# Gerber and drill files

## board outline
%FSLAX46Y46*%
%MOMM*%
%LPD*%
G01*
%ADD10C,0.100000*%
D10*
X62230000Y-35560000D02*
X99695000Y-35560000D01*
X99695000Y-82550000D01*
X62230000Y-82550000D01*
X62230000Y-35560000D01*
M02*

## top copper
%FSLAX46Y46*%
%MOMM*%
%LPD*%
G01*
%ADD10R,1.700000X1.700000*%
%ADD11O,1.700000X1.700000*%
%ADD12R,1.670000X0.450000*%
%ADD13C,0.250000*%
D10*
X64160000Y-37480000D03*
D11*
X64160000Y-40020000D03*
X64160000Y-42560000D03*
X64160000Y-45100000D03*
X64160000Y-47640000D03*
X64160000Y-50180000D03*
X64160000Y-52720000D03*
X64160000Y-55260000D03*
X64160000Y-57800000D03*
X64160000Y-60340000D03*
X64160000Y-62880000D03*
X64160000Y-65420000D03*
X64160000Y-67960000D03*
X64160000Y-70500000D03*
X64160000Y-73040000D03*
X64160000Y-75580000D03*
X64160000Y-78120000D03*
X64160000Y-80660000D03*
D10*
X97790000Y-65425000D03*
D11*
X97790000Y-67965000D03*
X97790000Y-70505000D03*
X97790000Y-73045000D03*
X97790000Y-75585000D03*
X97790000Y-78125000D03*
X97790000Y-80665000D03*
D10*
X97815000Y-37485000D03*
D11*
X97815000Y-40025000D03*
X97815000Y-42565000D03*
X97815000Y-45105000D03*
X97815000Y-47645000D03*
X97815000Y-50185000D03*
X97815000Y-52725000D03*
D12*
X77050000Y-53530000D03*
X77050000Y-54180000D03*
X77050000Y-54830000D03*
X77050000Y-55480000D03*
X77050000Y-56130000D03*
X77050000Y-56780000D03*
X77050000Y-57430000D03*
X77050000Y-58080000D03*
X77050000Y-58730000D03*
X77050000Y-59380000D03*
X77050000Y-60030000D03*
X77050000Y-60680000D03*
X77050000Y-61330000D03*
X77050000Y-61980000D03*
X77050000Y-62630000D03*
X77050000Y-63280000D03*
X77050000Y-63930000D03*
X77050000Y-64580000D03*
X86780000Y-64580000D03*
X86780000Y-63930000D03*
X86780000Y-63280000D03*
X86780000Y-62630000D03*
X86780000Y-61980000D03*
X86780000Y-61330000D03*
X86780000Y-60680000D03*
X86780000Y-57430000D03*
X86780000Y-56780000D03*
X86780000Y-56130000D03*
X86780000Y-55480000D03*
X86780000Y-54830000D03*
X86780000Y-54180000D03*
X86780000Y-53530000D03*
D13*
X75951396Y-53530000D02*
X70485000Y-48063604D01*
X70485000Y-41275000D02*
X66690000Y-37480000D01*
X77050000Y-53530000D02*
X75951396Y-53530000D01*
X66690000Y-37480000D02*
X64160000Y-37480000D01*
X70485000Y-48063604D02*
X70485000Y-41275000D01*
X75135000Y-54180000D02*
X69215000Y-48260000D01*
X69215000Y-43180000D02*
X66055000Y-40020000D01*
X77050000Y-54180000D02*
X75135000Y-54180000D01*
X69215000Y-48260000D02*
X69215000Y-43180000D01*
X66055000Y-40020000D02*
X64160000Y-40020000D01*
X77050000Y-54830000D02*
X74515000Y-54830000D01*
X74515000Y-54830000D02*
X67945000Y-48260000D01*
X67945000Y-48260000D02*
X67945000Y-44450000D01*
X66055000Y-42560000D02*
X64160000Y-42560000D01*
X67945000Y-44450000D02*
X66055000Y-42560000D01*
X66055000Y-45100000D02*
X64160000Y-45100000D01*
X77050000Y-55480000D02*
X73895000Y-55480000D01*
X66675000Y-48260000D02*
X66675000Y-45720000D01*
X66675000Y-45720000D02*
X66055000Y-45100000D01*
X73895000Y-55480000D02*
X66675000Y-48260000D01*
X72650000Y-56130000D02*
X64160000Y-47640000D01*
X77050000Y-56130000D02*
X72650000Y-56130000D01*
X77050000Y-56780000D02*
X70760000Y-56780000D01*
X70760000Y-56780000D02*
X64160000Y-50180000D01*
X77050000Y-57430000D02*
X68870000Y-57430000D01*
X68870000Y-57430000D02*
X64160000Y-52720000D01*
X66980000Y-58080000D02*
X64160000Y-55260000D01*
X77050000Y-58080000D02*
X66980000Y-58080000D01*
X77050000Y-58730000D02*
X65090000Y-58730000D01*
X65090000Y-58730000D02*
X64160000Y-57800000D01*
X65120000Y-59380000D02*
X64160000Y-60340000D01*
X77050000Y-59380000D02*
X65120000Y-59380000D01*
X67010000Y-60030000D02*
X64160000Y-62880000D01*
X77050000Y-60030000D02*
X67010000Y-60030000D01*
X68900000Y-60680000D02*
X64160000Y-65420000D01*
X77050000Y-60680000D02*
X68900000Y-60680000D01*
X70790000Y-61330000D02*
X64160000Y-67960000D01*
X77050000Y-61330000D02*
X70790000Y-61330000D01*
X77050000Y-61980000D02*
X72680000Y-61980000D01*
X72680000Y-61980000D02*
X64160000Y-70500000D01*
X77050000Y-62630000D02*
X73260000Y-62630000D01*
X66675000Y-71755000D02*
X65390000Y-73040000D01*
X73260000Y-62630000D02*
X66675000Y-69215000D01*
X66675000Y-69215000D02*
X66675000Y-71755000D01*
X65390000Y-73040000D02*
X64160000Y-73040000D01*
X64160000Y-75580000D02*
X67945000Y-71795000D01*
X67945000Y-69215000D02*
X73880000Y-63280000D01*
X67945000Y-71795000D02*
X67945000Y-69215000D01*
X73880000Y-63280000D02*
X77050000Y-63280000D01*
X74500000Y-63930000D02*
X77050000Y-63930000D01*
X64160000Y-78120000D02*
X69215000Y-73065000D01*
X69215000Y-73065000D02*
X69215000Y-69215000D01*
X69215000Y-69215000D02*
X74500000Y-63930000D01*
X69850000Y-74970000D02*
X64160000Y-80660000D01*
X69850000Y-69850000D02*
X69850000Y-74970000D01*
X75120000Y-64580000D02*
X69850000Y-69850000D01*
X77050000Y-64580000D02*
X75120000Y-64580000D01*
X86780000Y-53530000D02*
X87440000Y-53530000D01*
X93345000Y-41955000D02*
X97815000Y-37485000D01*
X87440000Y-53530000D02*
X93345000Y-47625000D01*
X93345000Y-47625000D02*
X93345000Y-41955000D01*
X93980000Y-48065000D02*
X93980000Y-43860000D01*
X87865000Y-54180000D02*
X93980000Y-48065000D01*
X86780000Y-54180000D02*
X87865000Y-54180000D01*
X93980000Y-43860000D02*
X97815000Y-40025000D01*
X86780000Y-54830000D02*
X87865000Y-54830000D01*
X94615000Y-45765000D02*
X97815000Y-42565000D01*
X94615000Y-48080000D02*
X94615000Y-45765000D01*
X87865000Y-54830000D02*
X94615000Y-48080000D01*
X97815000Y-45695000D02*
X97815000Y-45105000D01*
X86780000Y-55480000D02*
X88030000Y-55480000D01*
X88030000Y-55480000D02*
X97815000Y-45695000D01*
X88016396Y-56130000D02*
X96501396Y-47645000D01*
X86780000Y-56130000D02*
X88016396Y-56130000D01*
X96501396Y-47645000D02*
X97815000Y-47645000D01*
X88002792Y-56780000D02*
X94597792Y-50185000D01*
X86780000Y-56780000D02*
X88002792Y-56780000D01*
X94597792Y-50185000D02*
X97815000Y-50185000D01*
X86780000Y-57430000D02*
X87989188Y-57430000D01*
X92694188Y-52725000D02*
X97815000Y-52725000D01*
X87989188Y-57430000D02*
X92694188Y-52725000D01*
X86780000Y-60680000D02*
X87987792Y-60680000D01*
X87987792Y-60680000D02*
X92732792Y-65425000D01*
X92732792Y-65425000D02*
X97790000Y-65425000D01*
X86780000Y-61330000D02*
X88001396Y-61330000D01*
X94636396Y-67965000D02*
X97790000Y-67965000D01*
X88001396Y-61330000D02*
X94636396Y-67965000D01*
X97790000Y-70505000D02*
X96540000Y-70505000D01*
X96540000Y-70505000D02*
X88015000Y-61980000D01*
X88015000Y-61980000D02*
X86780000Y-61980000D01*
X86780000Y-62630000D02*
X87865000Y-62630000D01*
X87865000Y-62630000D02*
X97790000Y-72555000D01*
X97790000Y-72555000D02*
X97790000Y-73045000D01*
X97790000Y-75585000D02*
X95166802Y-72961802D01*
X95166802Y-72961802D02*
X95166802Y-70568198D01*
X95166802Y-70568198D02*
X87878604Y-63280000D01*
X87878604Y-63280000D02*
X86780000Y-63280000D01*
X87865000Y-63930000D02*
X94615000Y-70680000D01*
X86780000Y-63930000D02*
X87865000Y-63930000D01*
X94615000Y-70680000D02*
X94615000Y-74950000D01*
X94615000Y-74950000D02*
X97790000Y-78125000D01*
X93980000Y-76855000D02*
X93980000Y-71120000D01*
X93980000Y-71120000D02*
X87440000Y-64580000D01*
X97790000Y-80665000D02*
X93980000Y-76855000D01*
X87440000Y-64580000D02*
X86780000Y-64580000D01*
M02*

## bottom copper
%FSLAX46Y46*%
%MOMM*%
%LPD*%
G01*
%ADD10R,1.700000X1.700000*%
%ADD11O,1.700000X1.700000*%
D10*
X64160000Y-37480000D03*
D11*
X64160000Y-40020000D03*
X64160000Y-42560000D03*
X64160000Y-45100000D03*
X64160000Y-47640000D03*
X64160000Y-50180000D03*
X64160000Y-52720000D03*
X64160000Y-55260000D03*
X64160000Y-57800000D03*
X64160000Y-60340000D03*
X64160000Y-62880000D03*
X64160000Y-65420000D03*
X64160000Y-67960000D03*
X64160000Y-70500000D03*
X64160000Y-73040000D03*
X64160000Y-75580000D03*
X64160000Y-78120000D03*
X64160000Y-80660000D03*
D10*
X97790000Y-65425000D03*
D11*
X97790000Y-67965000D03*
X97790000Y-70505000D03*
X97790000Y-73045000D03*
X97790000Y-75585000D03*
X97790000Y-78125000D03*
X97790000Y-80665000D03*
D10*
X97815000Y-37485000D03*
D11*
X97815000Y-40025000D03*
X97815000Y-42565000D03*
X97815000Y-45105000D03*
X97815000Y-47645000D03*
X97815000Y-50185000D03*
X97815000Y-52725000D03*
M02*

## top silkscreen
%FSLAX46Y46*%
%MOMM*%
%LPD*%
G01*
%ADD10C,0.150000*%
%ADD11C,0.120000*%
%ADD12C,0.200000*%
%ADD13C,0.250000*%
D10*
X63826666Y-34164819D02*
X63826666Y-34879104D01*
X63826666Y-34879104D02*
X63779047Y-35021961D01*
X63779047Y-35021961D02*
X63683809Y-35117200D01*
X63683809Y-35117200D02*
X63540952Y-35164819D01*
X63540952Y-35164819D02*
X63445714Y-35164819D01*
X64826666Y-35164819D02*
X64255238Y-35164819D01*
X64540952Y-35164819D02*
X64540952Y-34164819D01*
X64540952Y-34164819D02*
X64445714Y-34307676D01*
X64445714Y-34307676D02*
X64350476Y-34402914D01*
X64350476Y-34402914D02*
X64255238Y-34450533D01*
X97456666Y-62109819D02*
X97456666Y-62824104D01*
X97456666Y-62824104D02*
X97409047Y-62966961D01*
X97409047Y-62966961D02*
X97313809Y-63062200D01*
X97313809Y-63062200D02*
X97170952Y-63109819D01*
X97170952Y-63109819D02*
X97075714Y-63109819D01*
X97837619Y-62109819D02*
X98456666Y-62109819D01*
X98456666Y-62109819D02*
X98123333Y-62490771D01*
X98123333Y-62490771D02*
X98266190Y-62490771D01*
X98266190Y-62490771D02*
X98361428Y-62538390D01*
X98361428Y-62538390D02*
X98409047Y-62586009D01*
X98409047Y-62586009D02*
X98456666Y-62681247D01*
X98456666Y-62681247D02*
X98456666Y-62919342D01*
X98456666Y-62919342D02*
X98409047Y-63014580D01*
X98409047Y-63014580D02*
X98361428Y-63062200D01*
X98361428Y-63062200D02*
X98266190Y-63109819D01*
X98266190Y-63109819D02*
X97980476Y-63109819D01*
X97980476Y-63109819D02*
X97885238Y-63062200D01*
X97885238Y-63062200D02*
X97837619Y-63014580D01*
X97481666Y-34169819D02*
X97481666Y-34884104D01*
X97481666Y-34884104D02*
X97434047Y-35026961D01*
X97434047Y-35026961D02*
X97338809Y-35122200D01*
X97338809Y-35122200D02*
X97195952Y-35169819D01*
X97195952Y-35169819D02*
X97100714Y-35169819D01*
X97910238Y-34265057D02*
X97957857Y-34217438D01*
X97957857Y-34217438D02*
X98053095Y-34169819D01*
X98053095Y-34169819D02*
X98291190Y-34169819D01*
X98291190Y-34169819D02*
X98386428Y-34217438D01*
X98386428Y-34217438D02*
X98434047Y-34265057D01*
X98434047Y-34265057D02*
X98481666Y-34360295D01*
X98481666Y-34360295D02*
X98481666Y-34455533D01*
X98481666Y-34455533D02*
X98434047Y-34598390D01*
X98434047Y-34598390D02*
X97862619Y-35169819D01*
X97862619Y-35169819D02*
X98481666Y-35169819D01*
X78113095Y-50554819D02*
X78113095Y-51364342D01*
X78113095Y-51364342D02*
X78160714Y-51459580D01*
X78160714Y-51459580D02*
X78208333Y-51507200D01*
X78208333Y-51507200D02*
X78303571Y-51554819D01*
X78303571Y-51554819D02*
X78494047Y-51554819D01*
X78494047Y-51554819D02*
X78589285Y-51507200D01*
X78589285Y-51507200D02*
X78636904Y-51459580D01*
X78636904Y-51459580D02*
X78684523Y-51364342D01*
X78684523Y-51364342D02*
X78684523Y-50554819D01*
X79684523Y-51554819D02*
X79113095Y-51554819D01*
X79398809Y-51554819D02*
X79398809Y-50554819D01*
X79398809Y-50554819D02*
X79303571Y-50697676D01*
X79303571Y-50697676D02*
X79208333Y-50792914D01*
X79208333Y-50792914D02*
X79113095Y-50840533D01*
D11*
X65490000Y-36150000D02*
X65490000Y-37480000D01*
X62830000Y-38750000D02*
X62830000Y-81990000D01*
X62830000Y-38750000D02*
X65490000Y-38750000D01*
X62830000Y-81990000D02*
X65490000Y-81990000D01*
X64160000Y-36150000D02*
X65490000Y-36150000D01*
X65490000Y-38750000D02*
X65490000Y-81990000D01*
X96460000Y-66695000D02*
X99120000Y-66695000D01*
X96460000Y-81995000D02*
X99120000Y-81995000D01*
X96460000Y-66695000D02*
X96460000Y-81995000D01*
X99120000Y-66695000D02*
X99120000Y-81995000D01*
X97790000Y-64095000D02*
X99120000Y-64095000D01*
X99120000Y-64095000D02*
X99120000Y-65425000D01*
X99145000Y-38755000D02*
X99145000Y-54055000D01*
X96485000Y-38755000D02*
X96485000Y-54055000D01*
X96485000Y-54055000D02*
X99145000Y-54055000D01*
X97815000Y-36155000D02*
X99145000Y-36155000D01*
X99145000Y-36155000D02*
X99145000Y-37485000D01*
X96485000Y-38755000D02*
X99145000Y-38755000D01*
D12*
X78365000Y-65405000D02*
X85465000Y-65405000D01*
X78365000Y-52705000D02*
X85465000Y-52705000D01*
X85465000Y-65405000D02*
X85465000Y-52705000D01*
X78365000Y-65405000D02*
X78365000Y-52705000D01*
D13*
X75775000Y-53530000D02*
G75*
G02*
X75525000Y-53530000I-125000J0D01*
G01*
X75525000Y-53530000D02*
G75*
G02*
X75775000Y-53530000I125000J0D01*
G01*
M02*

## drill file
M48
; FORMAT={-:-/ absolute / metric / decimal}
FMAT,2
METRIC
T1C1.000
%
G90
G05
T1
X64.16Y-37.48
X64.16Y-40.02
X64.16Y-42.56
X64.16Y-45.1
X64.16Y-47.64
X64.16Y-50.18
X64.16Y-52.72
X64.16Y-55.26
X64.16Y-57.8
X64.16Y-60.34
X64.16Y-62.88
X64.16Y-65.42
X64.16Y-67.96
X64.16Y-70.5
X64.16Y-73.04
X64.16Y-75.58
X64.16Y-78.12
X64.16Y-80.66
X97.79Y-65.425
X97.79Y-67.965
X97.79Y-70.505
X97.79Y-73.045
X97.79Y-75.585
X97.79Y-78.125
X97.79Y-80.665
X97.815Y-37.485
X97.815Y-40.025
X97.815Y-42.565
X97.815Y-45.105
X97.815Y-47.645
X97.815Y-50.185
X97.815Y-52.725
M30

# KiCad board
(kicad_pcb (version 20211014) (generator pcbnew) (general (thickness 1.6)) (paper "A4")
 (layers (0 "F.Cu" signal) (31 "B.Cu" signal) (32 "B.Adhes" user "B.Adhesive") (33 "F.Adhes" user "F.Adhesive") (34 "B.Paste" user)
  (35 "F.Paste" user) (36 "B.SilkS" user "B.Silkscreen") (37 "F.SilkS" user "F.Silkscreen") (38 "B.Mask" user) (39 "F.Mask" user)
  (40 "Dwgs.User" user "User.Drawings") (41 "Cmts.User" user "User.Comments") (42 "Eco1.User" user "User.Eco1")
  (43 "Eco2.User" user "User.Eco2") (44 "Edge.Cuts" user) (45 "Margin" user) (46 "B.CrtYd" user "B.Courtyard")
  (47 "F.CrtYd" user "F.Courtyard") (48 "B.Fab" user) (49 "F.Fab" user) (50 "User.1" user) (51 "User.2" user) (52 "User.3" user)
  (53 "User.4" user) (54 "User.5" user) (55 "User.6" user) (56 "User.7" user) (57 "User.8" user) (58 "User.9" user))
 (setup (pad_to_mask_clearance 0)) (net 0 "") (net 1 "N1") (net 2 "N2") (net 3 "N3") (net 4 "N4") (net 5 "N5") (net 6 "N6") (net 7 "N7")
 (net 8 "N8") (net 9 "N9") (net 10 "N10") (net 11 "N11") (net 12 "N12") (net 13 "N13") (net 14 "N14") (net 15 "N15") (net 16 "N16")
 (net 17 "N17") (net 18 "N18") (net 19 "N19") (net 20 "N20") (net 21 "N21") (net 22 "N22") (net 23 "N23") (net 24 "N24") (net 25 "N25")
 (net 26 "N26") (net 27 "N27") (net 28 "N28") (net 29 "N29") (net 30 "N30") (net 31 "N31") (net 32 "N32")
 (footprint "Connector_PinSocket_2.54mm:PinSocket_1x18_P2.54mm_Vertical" (layer "F.Cu") (at 64.16 37.48)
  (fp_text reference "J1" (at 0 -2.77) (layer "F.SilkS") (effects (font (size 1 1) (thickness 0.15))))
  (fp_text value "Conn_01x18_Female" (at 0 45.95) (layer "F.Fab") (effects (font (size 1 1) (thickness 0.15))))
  (fp_line (start 1.33 -1.33) (end 1.33 0) (layer "F.SilkS") (width 0.12))
  (fp_line (start -1.33 1.27) (end -1.33 44.51) (layer "F.SilkS") (width 0.12))
  (fp_line (start -1.33 1.27) (end 1.33 1.27) (layer "F.SilkS") (width 0.12))
  (fp_line (start -1.33 44.51) (end 1.33 44.51) (layer "F.SilkS") (width 0.12))
  (fp_line (start 0 -1.33) (end 1.33 -1.33) (layer "F.SilkS") (width 0.12))
  (fp_line (start 1.33 1.27) (end 1.33 44.51) (layer "F.SilkS") (width 0.12))
  (pad "1" thru_hole rect (at 0 0) (size 1.7 1.7) (drill 1) (layers *.Cu *.Mask) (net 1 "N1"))
  (pad "2" thru_hole oval (at 0 2.54) (size 1.7 1.7) (drill 1) (layers *.Cu *.Mask) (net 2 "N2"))
  (pad "3" thru_hole oval (at 0 5.08) (size 1.7 1.7) (drill 1) (layers *.Cu *.Mask) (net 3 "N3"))
  (pad "4" thru_hole oval (at 0 7.62) (size 1.7 1.7) (drill 1) (layers *.Cu *.Mask) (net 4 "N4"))
  (pad "5" thru_hole oval (at 0 10.16) (size 1.7 1.7) (drill 1) (layers *.Cu *.Mask) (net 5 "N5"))
  (pad "6" thru_hole oval (at 0 12.7) (size 1.7 1.7) (drill 1) (layers *.Cu *.Mask) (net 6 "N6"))
  (pad "7" thru_hole oval (at 0 15.24) (size 1.7 1.7) (drill 1) (layers *.Cu *.Mask) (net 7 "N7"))
  (pad "8" thru_hole oval (at 0 17.78) (size 1.7 1.7) (drill 1) (layers *.Cu *.Mask) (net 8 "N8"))
  (pad "9" thru_hole oval (at 0 20.32) (size 1.7 1.7) (drill 1) (layers *.Cu *.Mask) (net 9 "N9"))
  (pad "10" thru_hole oval (at 0 22.86) (size 1.7 1.7) (drill 1) (layers *.Cu *.Mask) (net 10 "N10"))
  (pad "11" thru_hole oval (at 0 25.4) (size 1.7 1.7) (drill 1) (layers *.Cu *.Mask) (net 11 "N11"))
  (pad "12" thru_hole oval (at 0 27.94) (size 1.7 1.7) (drill 1) (layers *.Cu *.Mask) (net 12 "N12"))
  (pad "13" thru_hole oval (at 0 30.48) (size 1.7 1.7) (drill 1) (layers *.Cu *.Mask) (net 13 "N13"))
  (pad "14" thru_hole oval (at 0 33.02) (size 1.7 1.7) (drill 1) (layers *.Cu *.Mask) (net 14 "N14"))
  (pad "15" thru_hole oval (at 0 35.56) (size 1.7 1.7) (drill 1) (layers *.Cu *.Mask) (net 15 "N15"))
  (pad "16" thru_hole oval (at 0 38.1) (size 1.7 1.7) (drill 1) (layers *.Cu *.Mask) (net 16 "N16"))
  (pad "17" thru_hole oval (at 0 40.64) (size 1.7 1.7) (drill 1) (layers *.Cu *.Mask) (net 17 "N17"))
  (pad "18" thru_hole oval (at 0 43.18) (size 1.7 1.7) (drill 1) (layers *.Cu *.Mask) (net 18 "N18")))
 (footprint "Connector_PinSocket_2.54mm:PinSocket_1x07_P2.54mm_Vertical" (layer "F.Cu") (at 97.79 65.425)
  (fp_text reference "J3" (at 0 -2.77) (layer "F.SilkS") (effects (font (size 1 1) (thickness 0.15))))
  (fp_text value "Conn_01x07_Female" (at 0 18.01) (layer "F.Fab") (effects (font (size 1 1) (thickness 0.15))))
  (fp_line (start -1.33 1.27) (end 1.33 1.27) (layer "F.SilkS") (width 0.12))
  (fp_line (start -1.33 16.57) (end 1.33 16.57) (layer "F.SilkS") (width 0.12))
  (fp_line (start -1.33 1.27) (end -1.33 16.57) (layer "F.SilkS") (width 0.12))
  (fp_line (start 1.33 1.27) (end 1.33 16.57) (layer "F.SilkS") (width 0.12))
  (fp_line (start 0 -1.33) (end 1.33 -1.33) (layer "F.SilkS") (width 0.12))
  (fp_line (start 1.33 -1.33) (end 1.33 0) (layer "F.SilkS") (width 0.12))
  (pad "1" thru_hole rect (at 0 0) (size 1.7 1.7) (drill 1) (layers *.Cu *.Mask) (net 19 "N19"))
  (pad "2" thru_hole oval (at 0 2.54) (size 1.7 1.7) (drill 1) (layers *.Cu *.Mask) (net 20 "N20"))
  (pad "3" thru_hole oval (at 0 5.08) (size 1.7 1.7) (drill 1) (layers *.Cu *.Mask) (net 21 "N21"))
  (pad "4" thru_hole oval (at 0 7.62) (size 1.7 1.7) (drill 1) (layers *.Cu *.Mask) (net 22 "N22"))
  (pad "5" thru_hole oval (at 0 10.16) (size 1.7 1.7) (drill 1) (layers *.Cu *.Mask) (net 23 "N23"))
  (pad "6" thru_hole oval (at 0 12.7) (size 1.7 1.7) (drill 1) (layers *.Cu *.Mask) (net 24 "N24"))
  (pad "7" thru_hole oval (at 0 15.24) (size 1.7 1.7) (drill 1) (layers *.Cu *.Mask) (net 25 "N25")))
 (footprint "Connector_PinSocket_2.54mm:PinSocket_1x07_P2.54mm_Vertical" (layer "F.Cu") (at 97.815 37.485)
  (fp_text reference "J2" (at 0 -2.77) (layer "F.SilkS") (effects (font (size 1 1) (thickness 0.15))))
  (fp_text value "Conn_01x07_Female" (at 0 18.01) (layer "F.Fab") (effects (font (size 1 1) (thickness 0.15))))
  (fp_line (start 1.33 1.27) (end 1.33 16.57) (layer "F.SilkS") (width 0.12))
  (fp_line (start -1.33 1.27) (end -1.33 16.57) (layer "F.SilkS") (width 0.12))
  (fp_line (start -1.33 16.57) (end 1.33 16.57) (layer "F.SilkS") (width 0.12))
  (fp_line (start 0 -1.33) (end 1.33 -1.33) (layer "F.SilkS") (width 0.12))
  (fp_line (start 1.33 -1.33) (end 1.33 0) (layer "F.SilkS") (width 0.12))
  (fp_line (start -1.33 1.27) (end 1.33 1.27) (layer "F.SilkS") (width 0.12))
  (pad "1" thru_hole rect (at 0 0) (size 1.7 1.7) (drill 1) (layers *.Cu *.Mask) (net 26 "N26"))
  (pad "2" thru_hole oval (at 0 2.54) (size 1.7 1.7) (drill 1) (layers *.Cu *.Mask) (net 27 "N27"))
  (pad "3" thru_hole oval (at 0 5.08) (size 1.7 1.7) (drill 1) (layers *.Cu *.Mask) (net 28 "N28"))
  (pad "4" thru_hole oval (at 0 7.62) (size 1.7 1.7) (drill 1) (layers *.Cu *.Mask) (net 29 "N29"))
  (pad "5" thru_hole oval (at 0 10.16) (size 1.7 1.7) (drill 1) (layers *.Cu *.Mask) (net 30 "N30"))
  (pad "6" thru_hole oval (at 0 12.7) (size 1.7 1.7) (drill 1) (layers *.Cu *.Mask) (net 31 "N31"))
  (pad "7" thru_hole oval (at 0 15.24) (size 1.7 1.7) (drill 1) (layers *.Cu *.Mask) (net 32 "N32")))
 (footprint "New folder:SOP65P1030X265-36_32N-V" (layer "F.Cu") (at 81.915 59.055)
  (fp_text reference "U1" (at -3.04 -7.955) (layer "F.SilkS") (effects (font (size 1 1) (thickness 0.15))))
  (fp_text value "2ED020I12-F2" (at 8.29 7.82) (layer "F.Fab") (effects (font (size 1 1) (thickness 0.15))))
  (fp_line (start -3.55 6.35) (end 3.55 6.35) (layer "F.SilkS") (width 0.2))
  (fp_line (start -3.55 -6.35) (end 3.55 -6.35) (layer "F.SilkS") (width 0.2))
  (fp_line (start 3.55 6.35) (end 3.55 -6.35) (layer "F.SilkS") (width 0.2))
  (fp_line (start -3.55 6.35) (end -3.55 -6.35) (layer "F.SilkS") (width 0.2))
  (fp_circle (center -6.265 -5.525) (end -6.14 -5.525) (layer "F.SilkS") (width 0.25) (fill none))
  (pad "1" smd rect locked (at -4.865 -5.525) (size 1.67 0.45) (layers "F.Cu" "F.Paste" "F.Mask") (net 1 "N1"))
  (pad "2" smd rect locked (at -4.865 -4.875) (size 1.67 0.45) (layers "F.Cu" "F.Paste" "F.Mask") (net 2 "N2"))
  (pad "3" smd rect locked (at -4.865 -4.225) (size 1.67 0.45) (layers "F.Cu" "F.Paste" "F.Mask") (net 3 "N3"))
  (pad "4" smd rect locked (at -4.865 -3.575) (size 1.67 0.45) (layers "F.Cu" "F.Paste" "F.Mask") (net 4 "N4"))
  (pad "5" smd rect locked (at -4.865 -2.925) (size 1.67 0.45) (layers "F.Cu" "F.Paste" "F.Mask") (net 5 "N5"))
  (pad "6" smd rect locked (at -4.865 -2.275) (size 1.67 0.45) (layers "F.Cu" "F.Paste" "F.Mask") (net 6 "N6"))
  (pad "7" smd rect locked (at -4.865 -1.625) (size 1.67 0.45) (layers "F.Cu" "F.Paste" "F.Mask") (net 7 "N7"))
  (pad "8" smd rect locked (at -4.865 -0.975) (size 1.67 0.45) (layers "F.Cu" "F.Paste" "F.Mask") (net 8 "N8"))
  (pad "9" smd rect locked (at -4.865 -0.325) (size 1.67 0.45) (layers "F.Cu" "F.Paste" "F.Mask") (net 9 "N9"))
  (pad "10" smd rect locked (at -4.865 0.325) (size 1.67 0.45) (layers "F.Cu" "F.Paste" "F.Mask") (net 10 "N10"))
  (pad "11" smd rect locked (at -4.865 0.975) (size 1.67 0.45) (layers "F.Cu" "F.Paste" "F.Mask") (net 11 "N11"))
  (pad "12" smd rect locked (at -4.865 1.625) (size 1.67 0.45) (layers "F.Cu" "F.Paste" "F.Mask") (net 12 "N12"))
  (pad "13" smd rect locked (at -4.865 2.275) (size 1.67 0.45) (layers "F.Cu" "F.Paste" "F.Mask") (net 13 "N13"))
  (pad "14" smd rect locked (at -4.865 2.925) (size 1.67 0.45) (layers "F.Cu" "F.Paste" "F.Mask") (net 14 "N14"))
  (pad "15" smd rect locked (at -4.865 3.575) (size 1.67 0.45) (layers "F.Cu" "F.Paste" "F.Mask") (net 15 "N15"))
  (pad "16" smd rect locked (at -4.865 4.225) (size 1.67 0.45) (layers "F.Cu" "F.Paste" "F.Mask") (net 16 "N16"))
  (pad "17" smd rect locked (at -4.865 4.875) (size 1.67 0.45) (layers "F.Cu" "F.Paste" "F.Mask") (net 17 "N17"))
  (pad "18" smd rect locked (at -4.865 5.525) (size 1.67 0.45) (layers "F.Cu" "F.Paste" "F.Mask") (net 18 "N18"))
  (pad "19" smd rect locked (at 4.865 5.525) (size 1.67 0.45) (layers "F.Cu" "F.Paste" "F.Mask") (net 25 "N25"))
  (pad "20" smd rect locked (at 4.865 4.875) (size 1.67 0.45) (layers "F.Cu" "F.Paste" "F.Mask") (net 24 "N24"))
  (pad "21" smd rect locked (at 4.865 4.225) (size 1.67 0.45) (layers "F.Cu" "F.Paste" "F.Mask") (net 23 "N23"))
  (pad "22" smd rect locked (at 4.865 3.575) (size 1.67 0.45) (layers "F.Cu" "F.Paste" "F.Mask") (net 22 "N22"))
  (pad "23" smd rect locked (at 4.865 2.925) (size 1.67 0.45) (layers "F.Cu" "F.Paste" "F.Mask") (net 21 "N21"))
  (pad "24" smd rect locked (at 4.865 2.275) (size 1.67 0.45) (layers "F.Cu" "F.Paste" "F.Mask") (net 20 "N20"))
  (pad "25" smd rect locked (at 4.865 1.625) (size 1.67 0.45) (layers "F.Cu" "F.Paste" "F.Mask") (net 19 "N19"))
  (pad "30" smd rect locked (at 4.865 -1.625) (size 1.67 0.45) (layers "F.Cu" "F.Paste" "F.Mask") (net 32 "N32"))
  (pad "31" smd rect locked (at 4.865 -2.275) (size 1.67 0.45) (layers "F.Cu" "F.Paste" "F.Mask") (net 31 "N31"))
  (pad "32" smd rect locked (at 4.865 -2.925) (size 1.67 0.45) (layers "F.Cu" "F.Paste" "F.Mask") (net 30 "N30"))
  (pad "33" smd rect locked (at 4.865 -3.575) (size 1.67 0.45) (layers "F.Cu" "F.Paste" "F.Mask") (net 29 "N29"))
  (pad "34" smd rect locked (at 4.865 -4.225) (size 1.67 0.45) (layers "F.Cu" "F.Paste" "F.Mask") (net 28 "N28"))
  (pad "35" smd rect locked (at 4.865 -4.875) (size 1.67 0.45) (layers "F.Cu" "F.Paste" "F.Mask") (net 27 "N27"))
  (pad "36" smd rect locked (at 4.865 -5.525) (size 1.67 0.45) (layers "F.Cu" "F.Paste" "F.Mask") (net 26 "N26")))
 (gr_rect (start 62.23 35.56) (end 99.695 82.55) (layer "Edge.Cuts") (width 0.1) (fill none))
 (segment (start 75.951396 53.53) (end 70.485 48.063604) (width 0.25) (layer "F.Cu") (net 1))
 (segment (start 70.485 41.275) (end 66.69 37.48) (width 0.25) (layer "F.Cu") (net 1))
 (segment (start 77.05 53.53) (end 75.951396 53.53) (width 0.25) (layer "F.Cu") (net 1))
 (segment (start 66.69 37.48) (end 64.16 37.48) (width 0.25) (layer "F.Cu") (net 1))
 (segment (start 70.485 48.063604) (end 70.485 41.275) (width 0.25) (layer "F.Cu") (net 1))
 (segment (start 75.135 54.18) (end 69.215 48.26) (width 0.25) (layer "F.Cu") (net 2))
 (segment (start 69.215 43.18) (end 66.055 40.02) (width 0.25) (layer "F.Cu") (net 2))
 (segment (start 77.05 54.18) (end 75.135 54.18) (width 0.25) (layer "F.Cu") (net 2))
 (segment (start 69.215 48.26) (end 69.215 43.18) (width 0.25) (layer "F.Cu") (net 2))
 (segment (start 66.055 40.02) (end 64.16 40.02) (width 0.25) (layer "F.Cu") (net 2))
 (segment (start 77.05 54.83) (end 74.515 54.83) (width 0.25) (layer "F.Cu") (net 3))
 (segment (start 74.515 54.83) (end 67.945 48.26) (width 0.25) (layer "F.Cu") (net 3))
 (segment (start 67.945 48.26) (end 67.945 44.45) (width 0.25) (layer "F.Cu") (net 3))
 (segment (start 66.055 42.56) (end 64.16 42.56) (width 0.25) (layer "F.Cu") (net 3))
 (segment (start 67.945 44.45) (end 66.055 42.56) (width 0.25) (layer "F.Cu") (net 3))
 (segment (start 66.055 45.1) (end 64.16 45.1) (width 0.25) (layer "F.Cu") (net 4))
 (segment (start 77.05 55.48) (end 73.895 55.48) (width 0.25) (layer "F.Cu") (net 4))
 (segment (start 66.675 48.26) (end 66.675 45.72) (width 0.25) (layer "F.Cu") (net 4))
 (segment (start 66.675 45.72) (end 66.055 45.1) (width 0.25) (layer "F.Cu") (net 4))
 (segment (start 73.895 55.48) (end 66.675 48.26) (width 0.25) (layer "F.Cu") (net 4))
 (segment (start 72.65 56.13) (end 64.16 47.64) (width 0.25) (layer "F.Cu") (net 5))
 (segment (start 77.05 56.13) (end 72.65 56.13) (width 0.25) (layer "F.Cu") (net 5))
 (segment (start 77.05 56.78) (end 70.76 56.78) (width 0.25) (layer "F.Cu") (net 6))
 (segment (start 70.76 56.78) (end 64.16 50.18) (width 0.25) (layer "F.Cu") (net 6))
 (segment (start 77.05 57.43) (end 68.87 57.43) (width 0.25) (layer "F.Cu") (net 7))
 (segment (start 68.87 57.43) (end 64.16 52.72) (width 0.25) (layer "F.Cu") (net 7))
 (segment (start 66.98 58.08) (end 64.16 55.26) (width 0.25) (layer "F.Cu") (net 8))
 (segment (start 77.05 58.08) (end 66.98 58.08) (width 0.25) (layer "F.Cu") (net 8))
 (segment (start 77.05 58.73) (end 65.09 58.73) (width 0.25) (layer "F.Cu") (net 9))
 (segment (start 65.09 58.73) (end 64.16 57.8) (width 0.25) (layer "F.Cu") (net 9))
 (segment (start 65.12 59.38) (end 64.16 60.34) (width 0.25) (layer "F.Cu") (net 10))
 (segment (start 77.05 59.38) (end 65.12 59.38) (width 0.25) (layer "F.Cu") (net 10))
 (segment (start 67.01 60.03) (end 64.16 62.88) (width 0.25) (layer "F.Cu") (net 11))
 (segment (start 77.05 60.03) (end 67.01 60.03) (width 0.25) (layer "F.Cu") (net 11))
 (segment (start 68.9 60.68) (end 64.16 65.42) (width 0.25) (layer "F.Cu") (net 12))
 (segment (start 77.05 60.68) (end 68.9 60.68) (width 0.25) (layer "F.Cu") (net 12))
 (segment (start 70.79 61.33) (end 64.16 67.96) (width 0.25) (layer "F.Cu") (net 13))
 (segment (start 77.05 61.33) (end 70.79 61.33) (width 0.25) (layer "F.Cu") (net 13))
 (segment (start 77.05 61.98) (end 72.68 61.98) (width 0.25) (layer "F.Cu") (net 14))
 (segment (start 72.68 61.98) (end 64.16 70.5) (width 0.25) (layer "F.Cu") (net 14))
 (segment (start 77.05 62.63) (end 73.26 62.63) (width 0.25) (layer "F.Cu") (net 15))
 (segment (start 66.675 71.755) (end 65.39 73.04) (width 0.25) (layer "F.Cu") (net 15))
 (segment (start 73.26 62.63) (end 66.675 69.215) (width 0.25) (layer "F.Cu") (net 15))
 (segment (start 66.675 69.215) (end 66.675 71.755) (width 0.25) (layer "F.Cu") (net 15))
 (segment (start 65.39 73.04) (end 64.16 73.04) (width 0.25) (layer "F.Cu") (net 15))
 (segment (start 64.16 75.58) (end 67.945 71.795) (width 0.25) (layer "F.Cu") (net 16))
 (segment (start 67.945 69.215) (end 73.88 63.28) (width 0.25) (layer "F.Cu") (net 16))
 (segment (start 67.945 71.795) (end 67.945 69.215) (width 0.25) (layer "F.Cu") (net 16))
 (segment (start 73.88 63.28) (end 77.05 63.28) (width 0.25) (layer "F.Cu") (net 16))
 (segment (start 74.5 63.93) (end 77.05 63.93) (width 0.25) (layer "F.Cu") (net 17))
 (segment (start 64.16 78.12) (end 69.215 73.065) (width 0.25) (layer "F.Cu") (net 17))
 (segment (start 69.215 73.065) (end 69.215 69.215) (width 0.25) (layer "F.Cu") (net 17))
 (segment (start 69.215 69.215) (end 74.5 63.93) (width 0.25) (layer "F.Cu") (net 17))
 (segment (start 69.85 74.97) (end 64.16 80.66) (width 0.25) (layer "F.Cu") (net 18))
 (segment (start 69.85 69.85) (end 69.85 74.97) (width 0.25) (layer "F.Cu") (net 18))
 (segment (start 75.12 64.58) (end 69.85 69.85) (width 0.25) (layer "F.Cu") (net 18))
 (segment (start 77.05 64.58) (end 75.12 64.58) (width 0.25) (layer "F.Cu") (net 18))
 (segment (start 86.78 53.53) (end 87.44 53.53) (width 0.25) (layer "F.Cu") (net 26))
 (segment (start 93.345 41.955) (end 97.815 37.485) (width 0.25) (layer "F.Cu") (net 26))
 (segment (start 87.44 53.53) (end 93.345 47.625) (width 0.25) (layer "F.Cu") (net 26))
 (segment (start 93.345 47.625) (end 93.345 41.955) (width 0.25) (layer "F.Cu") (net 26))
 (segment (start 93.98 48.065) (end 93.98 43.86) (width 0.25) (layer "F.Cu") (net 27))
 (segment (start 87.865 54.18) (end 93.98 48.065) (width 0.25) (layer "F.Cu") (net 27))
 (segment (start 86.78 54.18) (end 87.865 54.18) (width 0.25) (layer "F.Cu") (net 27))
 (segment (start 93.98 43.86) (end 97.815 40.025) (width 0.25) (layer "F.Cu") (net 27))
 (segment (start 86.78 54.83) (end 87.865 54.83) (width 0.25) (layer "F.Cu") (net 28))
 (segment (start 94.615 45.765) (end 97.815 42.565) (width 0.25) (layer "F.Cu") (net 28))
 (segment (start 94.615 48.08) (end 94.615 45.765) (width 0.25) (layer "F.Cu") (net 28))
 (segment (start 87.865 54.83) (end 94.615 48.08) (width 0.25) (layer "F.Cu") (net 28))
 (segment (start 97.815 45.695) (end 97.815 45.105) (width 0.25) (layer "F.Cu") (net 29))
 (segment (start 86.78 55.48) (end 88.03 55.48) (width 0.25) (layer "F.Cu") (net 29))
 (segment (start 88.03 55.48) (end 97.815 45.695) (width 0.25) (layer "F.Cu") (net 29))
 (segment (start 88.016396 56.13) (end 96.501396 47.645) (width 0.25) (layer "F.Cu") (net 30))
 (segment (start 86.78 56.13) (end 88.016396 56.13) (width 0.25) (layer "F.Cu") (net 30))
 (segment (start 96.501396 47.645) (end 97.815 47.645) (width 0.25) (layer "F.Cu") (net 30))
 (segment (start 88.002792 56.78) (end 94.597792 50.185) (width 0.25) (layer "F.Cu") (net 31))
 (segment (start 86.78 56.78) (end 88.002792 56.78) (width 0.25) (layer "F.Cu") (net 31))
 (segment (start 94.597792 50.185) (end 97.815 50.185) (width 0.25) (layer "F.Cu") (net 31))
 (segment (start 86.78 57.43) (end 87.989188 57.43) (width 0.25) (layer "F.Cu") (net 32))
 (segment (start 92.694188 52.725) (end 97.815 52.725) (width 0.25) (layer "F.Cu") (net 32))
 (segment (start 87.989188 57.43) (end 92.694188 52.725) (width 0.25) (layer "F.Cu") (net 32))
 (segment (start 86.78 60.68) (end 87.987792 60.68) (width 0.25) (layer "F.Cu") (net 19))
 (segment (start 87.987792 60.68) (end 92.732792 65.425) (width 0.25) (layer "F.Cu") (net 19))
 (segment (start 92.732792 65.425) (end 97.79 65.425) (width 0.25) (layer "F.Cu") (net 19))
 (segment (start 86.78 61.33) (end 88.001396 61.33) (width 0.25) (layer "F.Cu") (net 20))
 (segment (start 94.636396 67.965) (end 97.79 67.965) (width 0.25) (layer "F.Cu") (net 20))
 (segment (start 88.001396 61.33) (end 94.636396 67.965) (width 0.25) (layer "F.Cu") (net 20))
 (segment (start 97.79 70.505) (end 96.54 70.505) (width 0.25) (layer "F.Cu") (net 21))
 (segment (start 96.54 70.505) (end 88.015 61.98) (width 0.25) (layer "F.Cu") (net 21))
 (segment (start 88.015 61.98) (end 86.78 61.98) (width 0.25) (layer "F.Cu") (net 21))
 (segment (start 86.78 62.63) (end 87.865 62.63) (width 0.25) (layer "F.Cu") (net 22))
 (segment (start 87.865 62.63) (end 97.79 72.555) (width 0.25) (layer "F.Cu") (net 22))
 (segment (start 97.79 72.555) (end 97.79 73.045) (width 0.25) (layer "F.Cu") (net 22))
 (segment (start 97.79 75.585) (end 95.166802 72.961802) (width 0.25) (layer "F.Cu") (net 23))
 (segment (start 95.166802 72.961802) (end 95.166802 70.568198) (width 0.25) (layer "F.Cu") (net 23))
 (segment (start 95.166802 70.568198) (end 87.878604 63.28) (width 0.25) (layer "F.Cu") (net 23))
 (segment (start 87.878604 63.28) (end 86.78 63.28) (width 0.25) (layer "F.Cu") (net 23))
 (segment (start 87.865 63.93) (end 94.615 70.68) (width 0.25) (layer "F.Cu") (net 24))
 (segment (start 86.78 63.93) (end 87.865 63.93) (width 0.25) (layer "F.Cu") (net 24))
 (segment (start 94.615 70.68) (end 94.615 74.95) (width 0.25) (layer "F.Cu") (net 24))
 (segment (start 94.615 74.95) (end 97.79 78.125) (width 0.25) (layer "F.Cu") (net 24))
 (segment (start 93.98 76.855) (end 93.98 71.12) (width 0.25) (layer "F.Cu") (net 25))
 (segment (start 93.98 71.12) (end 87.44 64.58) (width 0.25) (layer "F.Cu") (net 25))
 (segment (start 97.79 80.665) (end 93.98 76.855) (width 0.25) (layer "F.Cu") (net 25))
 (segment (start 87.44 64.58) (end 86.78 64.58) (width 0.25) (layer "F.Cu") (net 25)))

